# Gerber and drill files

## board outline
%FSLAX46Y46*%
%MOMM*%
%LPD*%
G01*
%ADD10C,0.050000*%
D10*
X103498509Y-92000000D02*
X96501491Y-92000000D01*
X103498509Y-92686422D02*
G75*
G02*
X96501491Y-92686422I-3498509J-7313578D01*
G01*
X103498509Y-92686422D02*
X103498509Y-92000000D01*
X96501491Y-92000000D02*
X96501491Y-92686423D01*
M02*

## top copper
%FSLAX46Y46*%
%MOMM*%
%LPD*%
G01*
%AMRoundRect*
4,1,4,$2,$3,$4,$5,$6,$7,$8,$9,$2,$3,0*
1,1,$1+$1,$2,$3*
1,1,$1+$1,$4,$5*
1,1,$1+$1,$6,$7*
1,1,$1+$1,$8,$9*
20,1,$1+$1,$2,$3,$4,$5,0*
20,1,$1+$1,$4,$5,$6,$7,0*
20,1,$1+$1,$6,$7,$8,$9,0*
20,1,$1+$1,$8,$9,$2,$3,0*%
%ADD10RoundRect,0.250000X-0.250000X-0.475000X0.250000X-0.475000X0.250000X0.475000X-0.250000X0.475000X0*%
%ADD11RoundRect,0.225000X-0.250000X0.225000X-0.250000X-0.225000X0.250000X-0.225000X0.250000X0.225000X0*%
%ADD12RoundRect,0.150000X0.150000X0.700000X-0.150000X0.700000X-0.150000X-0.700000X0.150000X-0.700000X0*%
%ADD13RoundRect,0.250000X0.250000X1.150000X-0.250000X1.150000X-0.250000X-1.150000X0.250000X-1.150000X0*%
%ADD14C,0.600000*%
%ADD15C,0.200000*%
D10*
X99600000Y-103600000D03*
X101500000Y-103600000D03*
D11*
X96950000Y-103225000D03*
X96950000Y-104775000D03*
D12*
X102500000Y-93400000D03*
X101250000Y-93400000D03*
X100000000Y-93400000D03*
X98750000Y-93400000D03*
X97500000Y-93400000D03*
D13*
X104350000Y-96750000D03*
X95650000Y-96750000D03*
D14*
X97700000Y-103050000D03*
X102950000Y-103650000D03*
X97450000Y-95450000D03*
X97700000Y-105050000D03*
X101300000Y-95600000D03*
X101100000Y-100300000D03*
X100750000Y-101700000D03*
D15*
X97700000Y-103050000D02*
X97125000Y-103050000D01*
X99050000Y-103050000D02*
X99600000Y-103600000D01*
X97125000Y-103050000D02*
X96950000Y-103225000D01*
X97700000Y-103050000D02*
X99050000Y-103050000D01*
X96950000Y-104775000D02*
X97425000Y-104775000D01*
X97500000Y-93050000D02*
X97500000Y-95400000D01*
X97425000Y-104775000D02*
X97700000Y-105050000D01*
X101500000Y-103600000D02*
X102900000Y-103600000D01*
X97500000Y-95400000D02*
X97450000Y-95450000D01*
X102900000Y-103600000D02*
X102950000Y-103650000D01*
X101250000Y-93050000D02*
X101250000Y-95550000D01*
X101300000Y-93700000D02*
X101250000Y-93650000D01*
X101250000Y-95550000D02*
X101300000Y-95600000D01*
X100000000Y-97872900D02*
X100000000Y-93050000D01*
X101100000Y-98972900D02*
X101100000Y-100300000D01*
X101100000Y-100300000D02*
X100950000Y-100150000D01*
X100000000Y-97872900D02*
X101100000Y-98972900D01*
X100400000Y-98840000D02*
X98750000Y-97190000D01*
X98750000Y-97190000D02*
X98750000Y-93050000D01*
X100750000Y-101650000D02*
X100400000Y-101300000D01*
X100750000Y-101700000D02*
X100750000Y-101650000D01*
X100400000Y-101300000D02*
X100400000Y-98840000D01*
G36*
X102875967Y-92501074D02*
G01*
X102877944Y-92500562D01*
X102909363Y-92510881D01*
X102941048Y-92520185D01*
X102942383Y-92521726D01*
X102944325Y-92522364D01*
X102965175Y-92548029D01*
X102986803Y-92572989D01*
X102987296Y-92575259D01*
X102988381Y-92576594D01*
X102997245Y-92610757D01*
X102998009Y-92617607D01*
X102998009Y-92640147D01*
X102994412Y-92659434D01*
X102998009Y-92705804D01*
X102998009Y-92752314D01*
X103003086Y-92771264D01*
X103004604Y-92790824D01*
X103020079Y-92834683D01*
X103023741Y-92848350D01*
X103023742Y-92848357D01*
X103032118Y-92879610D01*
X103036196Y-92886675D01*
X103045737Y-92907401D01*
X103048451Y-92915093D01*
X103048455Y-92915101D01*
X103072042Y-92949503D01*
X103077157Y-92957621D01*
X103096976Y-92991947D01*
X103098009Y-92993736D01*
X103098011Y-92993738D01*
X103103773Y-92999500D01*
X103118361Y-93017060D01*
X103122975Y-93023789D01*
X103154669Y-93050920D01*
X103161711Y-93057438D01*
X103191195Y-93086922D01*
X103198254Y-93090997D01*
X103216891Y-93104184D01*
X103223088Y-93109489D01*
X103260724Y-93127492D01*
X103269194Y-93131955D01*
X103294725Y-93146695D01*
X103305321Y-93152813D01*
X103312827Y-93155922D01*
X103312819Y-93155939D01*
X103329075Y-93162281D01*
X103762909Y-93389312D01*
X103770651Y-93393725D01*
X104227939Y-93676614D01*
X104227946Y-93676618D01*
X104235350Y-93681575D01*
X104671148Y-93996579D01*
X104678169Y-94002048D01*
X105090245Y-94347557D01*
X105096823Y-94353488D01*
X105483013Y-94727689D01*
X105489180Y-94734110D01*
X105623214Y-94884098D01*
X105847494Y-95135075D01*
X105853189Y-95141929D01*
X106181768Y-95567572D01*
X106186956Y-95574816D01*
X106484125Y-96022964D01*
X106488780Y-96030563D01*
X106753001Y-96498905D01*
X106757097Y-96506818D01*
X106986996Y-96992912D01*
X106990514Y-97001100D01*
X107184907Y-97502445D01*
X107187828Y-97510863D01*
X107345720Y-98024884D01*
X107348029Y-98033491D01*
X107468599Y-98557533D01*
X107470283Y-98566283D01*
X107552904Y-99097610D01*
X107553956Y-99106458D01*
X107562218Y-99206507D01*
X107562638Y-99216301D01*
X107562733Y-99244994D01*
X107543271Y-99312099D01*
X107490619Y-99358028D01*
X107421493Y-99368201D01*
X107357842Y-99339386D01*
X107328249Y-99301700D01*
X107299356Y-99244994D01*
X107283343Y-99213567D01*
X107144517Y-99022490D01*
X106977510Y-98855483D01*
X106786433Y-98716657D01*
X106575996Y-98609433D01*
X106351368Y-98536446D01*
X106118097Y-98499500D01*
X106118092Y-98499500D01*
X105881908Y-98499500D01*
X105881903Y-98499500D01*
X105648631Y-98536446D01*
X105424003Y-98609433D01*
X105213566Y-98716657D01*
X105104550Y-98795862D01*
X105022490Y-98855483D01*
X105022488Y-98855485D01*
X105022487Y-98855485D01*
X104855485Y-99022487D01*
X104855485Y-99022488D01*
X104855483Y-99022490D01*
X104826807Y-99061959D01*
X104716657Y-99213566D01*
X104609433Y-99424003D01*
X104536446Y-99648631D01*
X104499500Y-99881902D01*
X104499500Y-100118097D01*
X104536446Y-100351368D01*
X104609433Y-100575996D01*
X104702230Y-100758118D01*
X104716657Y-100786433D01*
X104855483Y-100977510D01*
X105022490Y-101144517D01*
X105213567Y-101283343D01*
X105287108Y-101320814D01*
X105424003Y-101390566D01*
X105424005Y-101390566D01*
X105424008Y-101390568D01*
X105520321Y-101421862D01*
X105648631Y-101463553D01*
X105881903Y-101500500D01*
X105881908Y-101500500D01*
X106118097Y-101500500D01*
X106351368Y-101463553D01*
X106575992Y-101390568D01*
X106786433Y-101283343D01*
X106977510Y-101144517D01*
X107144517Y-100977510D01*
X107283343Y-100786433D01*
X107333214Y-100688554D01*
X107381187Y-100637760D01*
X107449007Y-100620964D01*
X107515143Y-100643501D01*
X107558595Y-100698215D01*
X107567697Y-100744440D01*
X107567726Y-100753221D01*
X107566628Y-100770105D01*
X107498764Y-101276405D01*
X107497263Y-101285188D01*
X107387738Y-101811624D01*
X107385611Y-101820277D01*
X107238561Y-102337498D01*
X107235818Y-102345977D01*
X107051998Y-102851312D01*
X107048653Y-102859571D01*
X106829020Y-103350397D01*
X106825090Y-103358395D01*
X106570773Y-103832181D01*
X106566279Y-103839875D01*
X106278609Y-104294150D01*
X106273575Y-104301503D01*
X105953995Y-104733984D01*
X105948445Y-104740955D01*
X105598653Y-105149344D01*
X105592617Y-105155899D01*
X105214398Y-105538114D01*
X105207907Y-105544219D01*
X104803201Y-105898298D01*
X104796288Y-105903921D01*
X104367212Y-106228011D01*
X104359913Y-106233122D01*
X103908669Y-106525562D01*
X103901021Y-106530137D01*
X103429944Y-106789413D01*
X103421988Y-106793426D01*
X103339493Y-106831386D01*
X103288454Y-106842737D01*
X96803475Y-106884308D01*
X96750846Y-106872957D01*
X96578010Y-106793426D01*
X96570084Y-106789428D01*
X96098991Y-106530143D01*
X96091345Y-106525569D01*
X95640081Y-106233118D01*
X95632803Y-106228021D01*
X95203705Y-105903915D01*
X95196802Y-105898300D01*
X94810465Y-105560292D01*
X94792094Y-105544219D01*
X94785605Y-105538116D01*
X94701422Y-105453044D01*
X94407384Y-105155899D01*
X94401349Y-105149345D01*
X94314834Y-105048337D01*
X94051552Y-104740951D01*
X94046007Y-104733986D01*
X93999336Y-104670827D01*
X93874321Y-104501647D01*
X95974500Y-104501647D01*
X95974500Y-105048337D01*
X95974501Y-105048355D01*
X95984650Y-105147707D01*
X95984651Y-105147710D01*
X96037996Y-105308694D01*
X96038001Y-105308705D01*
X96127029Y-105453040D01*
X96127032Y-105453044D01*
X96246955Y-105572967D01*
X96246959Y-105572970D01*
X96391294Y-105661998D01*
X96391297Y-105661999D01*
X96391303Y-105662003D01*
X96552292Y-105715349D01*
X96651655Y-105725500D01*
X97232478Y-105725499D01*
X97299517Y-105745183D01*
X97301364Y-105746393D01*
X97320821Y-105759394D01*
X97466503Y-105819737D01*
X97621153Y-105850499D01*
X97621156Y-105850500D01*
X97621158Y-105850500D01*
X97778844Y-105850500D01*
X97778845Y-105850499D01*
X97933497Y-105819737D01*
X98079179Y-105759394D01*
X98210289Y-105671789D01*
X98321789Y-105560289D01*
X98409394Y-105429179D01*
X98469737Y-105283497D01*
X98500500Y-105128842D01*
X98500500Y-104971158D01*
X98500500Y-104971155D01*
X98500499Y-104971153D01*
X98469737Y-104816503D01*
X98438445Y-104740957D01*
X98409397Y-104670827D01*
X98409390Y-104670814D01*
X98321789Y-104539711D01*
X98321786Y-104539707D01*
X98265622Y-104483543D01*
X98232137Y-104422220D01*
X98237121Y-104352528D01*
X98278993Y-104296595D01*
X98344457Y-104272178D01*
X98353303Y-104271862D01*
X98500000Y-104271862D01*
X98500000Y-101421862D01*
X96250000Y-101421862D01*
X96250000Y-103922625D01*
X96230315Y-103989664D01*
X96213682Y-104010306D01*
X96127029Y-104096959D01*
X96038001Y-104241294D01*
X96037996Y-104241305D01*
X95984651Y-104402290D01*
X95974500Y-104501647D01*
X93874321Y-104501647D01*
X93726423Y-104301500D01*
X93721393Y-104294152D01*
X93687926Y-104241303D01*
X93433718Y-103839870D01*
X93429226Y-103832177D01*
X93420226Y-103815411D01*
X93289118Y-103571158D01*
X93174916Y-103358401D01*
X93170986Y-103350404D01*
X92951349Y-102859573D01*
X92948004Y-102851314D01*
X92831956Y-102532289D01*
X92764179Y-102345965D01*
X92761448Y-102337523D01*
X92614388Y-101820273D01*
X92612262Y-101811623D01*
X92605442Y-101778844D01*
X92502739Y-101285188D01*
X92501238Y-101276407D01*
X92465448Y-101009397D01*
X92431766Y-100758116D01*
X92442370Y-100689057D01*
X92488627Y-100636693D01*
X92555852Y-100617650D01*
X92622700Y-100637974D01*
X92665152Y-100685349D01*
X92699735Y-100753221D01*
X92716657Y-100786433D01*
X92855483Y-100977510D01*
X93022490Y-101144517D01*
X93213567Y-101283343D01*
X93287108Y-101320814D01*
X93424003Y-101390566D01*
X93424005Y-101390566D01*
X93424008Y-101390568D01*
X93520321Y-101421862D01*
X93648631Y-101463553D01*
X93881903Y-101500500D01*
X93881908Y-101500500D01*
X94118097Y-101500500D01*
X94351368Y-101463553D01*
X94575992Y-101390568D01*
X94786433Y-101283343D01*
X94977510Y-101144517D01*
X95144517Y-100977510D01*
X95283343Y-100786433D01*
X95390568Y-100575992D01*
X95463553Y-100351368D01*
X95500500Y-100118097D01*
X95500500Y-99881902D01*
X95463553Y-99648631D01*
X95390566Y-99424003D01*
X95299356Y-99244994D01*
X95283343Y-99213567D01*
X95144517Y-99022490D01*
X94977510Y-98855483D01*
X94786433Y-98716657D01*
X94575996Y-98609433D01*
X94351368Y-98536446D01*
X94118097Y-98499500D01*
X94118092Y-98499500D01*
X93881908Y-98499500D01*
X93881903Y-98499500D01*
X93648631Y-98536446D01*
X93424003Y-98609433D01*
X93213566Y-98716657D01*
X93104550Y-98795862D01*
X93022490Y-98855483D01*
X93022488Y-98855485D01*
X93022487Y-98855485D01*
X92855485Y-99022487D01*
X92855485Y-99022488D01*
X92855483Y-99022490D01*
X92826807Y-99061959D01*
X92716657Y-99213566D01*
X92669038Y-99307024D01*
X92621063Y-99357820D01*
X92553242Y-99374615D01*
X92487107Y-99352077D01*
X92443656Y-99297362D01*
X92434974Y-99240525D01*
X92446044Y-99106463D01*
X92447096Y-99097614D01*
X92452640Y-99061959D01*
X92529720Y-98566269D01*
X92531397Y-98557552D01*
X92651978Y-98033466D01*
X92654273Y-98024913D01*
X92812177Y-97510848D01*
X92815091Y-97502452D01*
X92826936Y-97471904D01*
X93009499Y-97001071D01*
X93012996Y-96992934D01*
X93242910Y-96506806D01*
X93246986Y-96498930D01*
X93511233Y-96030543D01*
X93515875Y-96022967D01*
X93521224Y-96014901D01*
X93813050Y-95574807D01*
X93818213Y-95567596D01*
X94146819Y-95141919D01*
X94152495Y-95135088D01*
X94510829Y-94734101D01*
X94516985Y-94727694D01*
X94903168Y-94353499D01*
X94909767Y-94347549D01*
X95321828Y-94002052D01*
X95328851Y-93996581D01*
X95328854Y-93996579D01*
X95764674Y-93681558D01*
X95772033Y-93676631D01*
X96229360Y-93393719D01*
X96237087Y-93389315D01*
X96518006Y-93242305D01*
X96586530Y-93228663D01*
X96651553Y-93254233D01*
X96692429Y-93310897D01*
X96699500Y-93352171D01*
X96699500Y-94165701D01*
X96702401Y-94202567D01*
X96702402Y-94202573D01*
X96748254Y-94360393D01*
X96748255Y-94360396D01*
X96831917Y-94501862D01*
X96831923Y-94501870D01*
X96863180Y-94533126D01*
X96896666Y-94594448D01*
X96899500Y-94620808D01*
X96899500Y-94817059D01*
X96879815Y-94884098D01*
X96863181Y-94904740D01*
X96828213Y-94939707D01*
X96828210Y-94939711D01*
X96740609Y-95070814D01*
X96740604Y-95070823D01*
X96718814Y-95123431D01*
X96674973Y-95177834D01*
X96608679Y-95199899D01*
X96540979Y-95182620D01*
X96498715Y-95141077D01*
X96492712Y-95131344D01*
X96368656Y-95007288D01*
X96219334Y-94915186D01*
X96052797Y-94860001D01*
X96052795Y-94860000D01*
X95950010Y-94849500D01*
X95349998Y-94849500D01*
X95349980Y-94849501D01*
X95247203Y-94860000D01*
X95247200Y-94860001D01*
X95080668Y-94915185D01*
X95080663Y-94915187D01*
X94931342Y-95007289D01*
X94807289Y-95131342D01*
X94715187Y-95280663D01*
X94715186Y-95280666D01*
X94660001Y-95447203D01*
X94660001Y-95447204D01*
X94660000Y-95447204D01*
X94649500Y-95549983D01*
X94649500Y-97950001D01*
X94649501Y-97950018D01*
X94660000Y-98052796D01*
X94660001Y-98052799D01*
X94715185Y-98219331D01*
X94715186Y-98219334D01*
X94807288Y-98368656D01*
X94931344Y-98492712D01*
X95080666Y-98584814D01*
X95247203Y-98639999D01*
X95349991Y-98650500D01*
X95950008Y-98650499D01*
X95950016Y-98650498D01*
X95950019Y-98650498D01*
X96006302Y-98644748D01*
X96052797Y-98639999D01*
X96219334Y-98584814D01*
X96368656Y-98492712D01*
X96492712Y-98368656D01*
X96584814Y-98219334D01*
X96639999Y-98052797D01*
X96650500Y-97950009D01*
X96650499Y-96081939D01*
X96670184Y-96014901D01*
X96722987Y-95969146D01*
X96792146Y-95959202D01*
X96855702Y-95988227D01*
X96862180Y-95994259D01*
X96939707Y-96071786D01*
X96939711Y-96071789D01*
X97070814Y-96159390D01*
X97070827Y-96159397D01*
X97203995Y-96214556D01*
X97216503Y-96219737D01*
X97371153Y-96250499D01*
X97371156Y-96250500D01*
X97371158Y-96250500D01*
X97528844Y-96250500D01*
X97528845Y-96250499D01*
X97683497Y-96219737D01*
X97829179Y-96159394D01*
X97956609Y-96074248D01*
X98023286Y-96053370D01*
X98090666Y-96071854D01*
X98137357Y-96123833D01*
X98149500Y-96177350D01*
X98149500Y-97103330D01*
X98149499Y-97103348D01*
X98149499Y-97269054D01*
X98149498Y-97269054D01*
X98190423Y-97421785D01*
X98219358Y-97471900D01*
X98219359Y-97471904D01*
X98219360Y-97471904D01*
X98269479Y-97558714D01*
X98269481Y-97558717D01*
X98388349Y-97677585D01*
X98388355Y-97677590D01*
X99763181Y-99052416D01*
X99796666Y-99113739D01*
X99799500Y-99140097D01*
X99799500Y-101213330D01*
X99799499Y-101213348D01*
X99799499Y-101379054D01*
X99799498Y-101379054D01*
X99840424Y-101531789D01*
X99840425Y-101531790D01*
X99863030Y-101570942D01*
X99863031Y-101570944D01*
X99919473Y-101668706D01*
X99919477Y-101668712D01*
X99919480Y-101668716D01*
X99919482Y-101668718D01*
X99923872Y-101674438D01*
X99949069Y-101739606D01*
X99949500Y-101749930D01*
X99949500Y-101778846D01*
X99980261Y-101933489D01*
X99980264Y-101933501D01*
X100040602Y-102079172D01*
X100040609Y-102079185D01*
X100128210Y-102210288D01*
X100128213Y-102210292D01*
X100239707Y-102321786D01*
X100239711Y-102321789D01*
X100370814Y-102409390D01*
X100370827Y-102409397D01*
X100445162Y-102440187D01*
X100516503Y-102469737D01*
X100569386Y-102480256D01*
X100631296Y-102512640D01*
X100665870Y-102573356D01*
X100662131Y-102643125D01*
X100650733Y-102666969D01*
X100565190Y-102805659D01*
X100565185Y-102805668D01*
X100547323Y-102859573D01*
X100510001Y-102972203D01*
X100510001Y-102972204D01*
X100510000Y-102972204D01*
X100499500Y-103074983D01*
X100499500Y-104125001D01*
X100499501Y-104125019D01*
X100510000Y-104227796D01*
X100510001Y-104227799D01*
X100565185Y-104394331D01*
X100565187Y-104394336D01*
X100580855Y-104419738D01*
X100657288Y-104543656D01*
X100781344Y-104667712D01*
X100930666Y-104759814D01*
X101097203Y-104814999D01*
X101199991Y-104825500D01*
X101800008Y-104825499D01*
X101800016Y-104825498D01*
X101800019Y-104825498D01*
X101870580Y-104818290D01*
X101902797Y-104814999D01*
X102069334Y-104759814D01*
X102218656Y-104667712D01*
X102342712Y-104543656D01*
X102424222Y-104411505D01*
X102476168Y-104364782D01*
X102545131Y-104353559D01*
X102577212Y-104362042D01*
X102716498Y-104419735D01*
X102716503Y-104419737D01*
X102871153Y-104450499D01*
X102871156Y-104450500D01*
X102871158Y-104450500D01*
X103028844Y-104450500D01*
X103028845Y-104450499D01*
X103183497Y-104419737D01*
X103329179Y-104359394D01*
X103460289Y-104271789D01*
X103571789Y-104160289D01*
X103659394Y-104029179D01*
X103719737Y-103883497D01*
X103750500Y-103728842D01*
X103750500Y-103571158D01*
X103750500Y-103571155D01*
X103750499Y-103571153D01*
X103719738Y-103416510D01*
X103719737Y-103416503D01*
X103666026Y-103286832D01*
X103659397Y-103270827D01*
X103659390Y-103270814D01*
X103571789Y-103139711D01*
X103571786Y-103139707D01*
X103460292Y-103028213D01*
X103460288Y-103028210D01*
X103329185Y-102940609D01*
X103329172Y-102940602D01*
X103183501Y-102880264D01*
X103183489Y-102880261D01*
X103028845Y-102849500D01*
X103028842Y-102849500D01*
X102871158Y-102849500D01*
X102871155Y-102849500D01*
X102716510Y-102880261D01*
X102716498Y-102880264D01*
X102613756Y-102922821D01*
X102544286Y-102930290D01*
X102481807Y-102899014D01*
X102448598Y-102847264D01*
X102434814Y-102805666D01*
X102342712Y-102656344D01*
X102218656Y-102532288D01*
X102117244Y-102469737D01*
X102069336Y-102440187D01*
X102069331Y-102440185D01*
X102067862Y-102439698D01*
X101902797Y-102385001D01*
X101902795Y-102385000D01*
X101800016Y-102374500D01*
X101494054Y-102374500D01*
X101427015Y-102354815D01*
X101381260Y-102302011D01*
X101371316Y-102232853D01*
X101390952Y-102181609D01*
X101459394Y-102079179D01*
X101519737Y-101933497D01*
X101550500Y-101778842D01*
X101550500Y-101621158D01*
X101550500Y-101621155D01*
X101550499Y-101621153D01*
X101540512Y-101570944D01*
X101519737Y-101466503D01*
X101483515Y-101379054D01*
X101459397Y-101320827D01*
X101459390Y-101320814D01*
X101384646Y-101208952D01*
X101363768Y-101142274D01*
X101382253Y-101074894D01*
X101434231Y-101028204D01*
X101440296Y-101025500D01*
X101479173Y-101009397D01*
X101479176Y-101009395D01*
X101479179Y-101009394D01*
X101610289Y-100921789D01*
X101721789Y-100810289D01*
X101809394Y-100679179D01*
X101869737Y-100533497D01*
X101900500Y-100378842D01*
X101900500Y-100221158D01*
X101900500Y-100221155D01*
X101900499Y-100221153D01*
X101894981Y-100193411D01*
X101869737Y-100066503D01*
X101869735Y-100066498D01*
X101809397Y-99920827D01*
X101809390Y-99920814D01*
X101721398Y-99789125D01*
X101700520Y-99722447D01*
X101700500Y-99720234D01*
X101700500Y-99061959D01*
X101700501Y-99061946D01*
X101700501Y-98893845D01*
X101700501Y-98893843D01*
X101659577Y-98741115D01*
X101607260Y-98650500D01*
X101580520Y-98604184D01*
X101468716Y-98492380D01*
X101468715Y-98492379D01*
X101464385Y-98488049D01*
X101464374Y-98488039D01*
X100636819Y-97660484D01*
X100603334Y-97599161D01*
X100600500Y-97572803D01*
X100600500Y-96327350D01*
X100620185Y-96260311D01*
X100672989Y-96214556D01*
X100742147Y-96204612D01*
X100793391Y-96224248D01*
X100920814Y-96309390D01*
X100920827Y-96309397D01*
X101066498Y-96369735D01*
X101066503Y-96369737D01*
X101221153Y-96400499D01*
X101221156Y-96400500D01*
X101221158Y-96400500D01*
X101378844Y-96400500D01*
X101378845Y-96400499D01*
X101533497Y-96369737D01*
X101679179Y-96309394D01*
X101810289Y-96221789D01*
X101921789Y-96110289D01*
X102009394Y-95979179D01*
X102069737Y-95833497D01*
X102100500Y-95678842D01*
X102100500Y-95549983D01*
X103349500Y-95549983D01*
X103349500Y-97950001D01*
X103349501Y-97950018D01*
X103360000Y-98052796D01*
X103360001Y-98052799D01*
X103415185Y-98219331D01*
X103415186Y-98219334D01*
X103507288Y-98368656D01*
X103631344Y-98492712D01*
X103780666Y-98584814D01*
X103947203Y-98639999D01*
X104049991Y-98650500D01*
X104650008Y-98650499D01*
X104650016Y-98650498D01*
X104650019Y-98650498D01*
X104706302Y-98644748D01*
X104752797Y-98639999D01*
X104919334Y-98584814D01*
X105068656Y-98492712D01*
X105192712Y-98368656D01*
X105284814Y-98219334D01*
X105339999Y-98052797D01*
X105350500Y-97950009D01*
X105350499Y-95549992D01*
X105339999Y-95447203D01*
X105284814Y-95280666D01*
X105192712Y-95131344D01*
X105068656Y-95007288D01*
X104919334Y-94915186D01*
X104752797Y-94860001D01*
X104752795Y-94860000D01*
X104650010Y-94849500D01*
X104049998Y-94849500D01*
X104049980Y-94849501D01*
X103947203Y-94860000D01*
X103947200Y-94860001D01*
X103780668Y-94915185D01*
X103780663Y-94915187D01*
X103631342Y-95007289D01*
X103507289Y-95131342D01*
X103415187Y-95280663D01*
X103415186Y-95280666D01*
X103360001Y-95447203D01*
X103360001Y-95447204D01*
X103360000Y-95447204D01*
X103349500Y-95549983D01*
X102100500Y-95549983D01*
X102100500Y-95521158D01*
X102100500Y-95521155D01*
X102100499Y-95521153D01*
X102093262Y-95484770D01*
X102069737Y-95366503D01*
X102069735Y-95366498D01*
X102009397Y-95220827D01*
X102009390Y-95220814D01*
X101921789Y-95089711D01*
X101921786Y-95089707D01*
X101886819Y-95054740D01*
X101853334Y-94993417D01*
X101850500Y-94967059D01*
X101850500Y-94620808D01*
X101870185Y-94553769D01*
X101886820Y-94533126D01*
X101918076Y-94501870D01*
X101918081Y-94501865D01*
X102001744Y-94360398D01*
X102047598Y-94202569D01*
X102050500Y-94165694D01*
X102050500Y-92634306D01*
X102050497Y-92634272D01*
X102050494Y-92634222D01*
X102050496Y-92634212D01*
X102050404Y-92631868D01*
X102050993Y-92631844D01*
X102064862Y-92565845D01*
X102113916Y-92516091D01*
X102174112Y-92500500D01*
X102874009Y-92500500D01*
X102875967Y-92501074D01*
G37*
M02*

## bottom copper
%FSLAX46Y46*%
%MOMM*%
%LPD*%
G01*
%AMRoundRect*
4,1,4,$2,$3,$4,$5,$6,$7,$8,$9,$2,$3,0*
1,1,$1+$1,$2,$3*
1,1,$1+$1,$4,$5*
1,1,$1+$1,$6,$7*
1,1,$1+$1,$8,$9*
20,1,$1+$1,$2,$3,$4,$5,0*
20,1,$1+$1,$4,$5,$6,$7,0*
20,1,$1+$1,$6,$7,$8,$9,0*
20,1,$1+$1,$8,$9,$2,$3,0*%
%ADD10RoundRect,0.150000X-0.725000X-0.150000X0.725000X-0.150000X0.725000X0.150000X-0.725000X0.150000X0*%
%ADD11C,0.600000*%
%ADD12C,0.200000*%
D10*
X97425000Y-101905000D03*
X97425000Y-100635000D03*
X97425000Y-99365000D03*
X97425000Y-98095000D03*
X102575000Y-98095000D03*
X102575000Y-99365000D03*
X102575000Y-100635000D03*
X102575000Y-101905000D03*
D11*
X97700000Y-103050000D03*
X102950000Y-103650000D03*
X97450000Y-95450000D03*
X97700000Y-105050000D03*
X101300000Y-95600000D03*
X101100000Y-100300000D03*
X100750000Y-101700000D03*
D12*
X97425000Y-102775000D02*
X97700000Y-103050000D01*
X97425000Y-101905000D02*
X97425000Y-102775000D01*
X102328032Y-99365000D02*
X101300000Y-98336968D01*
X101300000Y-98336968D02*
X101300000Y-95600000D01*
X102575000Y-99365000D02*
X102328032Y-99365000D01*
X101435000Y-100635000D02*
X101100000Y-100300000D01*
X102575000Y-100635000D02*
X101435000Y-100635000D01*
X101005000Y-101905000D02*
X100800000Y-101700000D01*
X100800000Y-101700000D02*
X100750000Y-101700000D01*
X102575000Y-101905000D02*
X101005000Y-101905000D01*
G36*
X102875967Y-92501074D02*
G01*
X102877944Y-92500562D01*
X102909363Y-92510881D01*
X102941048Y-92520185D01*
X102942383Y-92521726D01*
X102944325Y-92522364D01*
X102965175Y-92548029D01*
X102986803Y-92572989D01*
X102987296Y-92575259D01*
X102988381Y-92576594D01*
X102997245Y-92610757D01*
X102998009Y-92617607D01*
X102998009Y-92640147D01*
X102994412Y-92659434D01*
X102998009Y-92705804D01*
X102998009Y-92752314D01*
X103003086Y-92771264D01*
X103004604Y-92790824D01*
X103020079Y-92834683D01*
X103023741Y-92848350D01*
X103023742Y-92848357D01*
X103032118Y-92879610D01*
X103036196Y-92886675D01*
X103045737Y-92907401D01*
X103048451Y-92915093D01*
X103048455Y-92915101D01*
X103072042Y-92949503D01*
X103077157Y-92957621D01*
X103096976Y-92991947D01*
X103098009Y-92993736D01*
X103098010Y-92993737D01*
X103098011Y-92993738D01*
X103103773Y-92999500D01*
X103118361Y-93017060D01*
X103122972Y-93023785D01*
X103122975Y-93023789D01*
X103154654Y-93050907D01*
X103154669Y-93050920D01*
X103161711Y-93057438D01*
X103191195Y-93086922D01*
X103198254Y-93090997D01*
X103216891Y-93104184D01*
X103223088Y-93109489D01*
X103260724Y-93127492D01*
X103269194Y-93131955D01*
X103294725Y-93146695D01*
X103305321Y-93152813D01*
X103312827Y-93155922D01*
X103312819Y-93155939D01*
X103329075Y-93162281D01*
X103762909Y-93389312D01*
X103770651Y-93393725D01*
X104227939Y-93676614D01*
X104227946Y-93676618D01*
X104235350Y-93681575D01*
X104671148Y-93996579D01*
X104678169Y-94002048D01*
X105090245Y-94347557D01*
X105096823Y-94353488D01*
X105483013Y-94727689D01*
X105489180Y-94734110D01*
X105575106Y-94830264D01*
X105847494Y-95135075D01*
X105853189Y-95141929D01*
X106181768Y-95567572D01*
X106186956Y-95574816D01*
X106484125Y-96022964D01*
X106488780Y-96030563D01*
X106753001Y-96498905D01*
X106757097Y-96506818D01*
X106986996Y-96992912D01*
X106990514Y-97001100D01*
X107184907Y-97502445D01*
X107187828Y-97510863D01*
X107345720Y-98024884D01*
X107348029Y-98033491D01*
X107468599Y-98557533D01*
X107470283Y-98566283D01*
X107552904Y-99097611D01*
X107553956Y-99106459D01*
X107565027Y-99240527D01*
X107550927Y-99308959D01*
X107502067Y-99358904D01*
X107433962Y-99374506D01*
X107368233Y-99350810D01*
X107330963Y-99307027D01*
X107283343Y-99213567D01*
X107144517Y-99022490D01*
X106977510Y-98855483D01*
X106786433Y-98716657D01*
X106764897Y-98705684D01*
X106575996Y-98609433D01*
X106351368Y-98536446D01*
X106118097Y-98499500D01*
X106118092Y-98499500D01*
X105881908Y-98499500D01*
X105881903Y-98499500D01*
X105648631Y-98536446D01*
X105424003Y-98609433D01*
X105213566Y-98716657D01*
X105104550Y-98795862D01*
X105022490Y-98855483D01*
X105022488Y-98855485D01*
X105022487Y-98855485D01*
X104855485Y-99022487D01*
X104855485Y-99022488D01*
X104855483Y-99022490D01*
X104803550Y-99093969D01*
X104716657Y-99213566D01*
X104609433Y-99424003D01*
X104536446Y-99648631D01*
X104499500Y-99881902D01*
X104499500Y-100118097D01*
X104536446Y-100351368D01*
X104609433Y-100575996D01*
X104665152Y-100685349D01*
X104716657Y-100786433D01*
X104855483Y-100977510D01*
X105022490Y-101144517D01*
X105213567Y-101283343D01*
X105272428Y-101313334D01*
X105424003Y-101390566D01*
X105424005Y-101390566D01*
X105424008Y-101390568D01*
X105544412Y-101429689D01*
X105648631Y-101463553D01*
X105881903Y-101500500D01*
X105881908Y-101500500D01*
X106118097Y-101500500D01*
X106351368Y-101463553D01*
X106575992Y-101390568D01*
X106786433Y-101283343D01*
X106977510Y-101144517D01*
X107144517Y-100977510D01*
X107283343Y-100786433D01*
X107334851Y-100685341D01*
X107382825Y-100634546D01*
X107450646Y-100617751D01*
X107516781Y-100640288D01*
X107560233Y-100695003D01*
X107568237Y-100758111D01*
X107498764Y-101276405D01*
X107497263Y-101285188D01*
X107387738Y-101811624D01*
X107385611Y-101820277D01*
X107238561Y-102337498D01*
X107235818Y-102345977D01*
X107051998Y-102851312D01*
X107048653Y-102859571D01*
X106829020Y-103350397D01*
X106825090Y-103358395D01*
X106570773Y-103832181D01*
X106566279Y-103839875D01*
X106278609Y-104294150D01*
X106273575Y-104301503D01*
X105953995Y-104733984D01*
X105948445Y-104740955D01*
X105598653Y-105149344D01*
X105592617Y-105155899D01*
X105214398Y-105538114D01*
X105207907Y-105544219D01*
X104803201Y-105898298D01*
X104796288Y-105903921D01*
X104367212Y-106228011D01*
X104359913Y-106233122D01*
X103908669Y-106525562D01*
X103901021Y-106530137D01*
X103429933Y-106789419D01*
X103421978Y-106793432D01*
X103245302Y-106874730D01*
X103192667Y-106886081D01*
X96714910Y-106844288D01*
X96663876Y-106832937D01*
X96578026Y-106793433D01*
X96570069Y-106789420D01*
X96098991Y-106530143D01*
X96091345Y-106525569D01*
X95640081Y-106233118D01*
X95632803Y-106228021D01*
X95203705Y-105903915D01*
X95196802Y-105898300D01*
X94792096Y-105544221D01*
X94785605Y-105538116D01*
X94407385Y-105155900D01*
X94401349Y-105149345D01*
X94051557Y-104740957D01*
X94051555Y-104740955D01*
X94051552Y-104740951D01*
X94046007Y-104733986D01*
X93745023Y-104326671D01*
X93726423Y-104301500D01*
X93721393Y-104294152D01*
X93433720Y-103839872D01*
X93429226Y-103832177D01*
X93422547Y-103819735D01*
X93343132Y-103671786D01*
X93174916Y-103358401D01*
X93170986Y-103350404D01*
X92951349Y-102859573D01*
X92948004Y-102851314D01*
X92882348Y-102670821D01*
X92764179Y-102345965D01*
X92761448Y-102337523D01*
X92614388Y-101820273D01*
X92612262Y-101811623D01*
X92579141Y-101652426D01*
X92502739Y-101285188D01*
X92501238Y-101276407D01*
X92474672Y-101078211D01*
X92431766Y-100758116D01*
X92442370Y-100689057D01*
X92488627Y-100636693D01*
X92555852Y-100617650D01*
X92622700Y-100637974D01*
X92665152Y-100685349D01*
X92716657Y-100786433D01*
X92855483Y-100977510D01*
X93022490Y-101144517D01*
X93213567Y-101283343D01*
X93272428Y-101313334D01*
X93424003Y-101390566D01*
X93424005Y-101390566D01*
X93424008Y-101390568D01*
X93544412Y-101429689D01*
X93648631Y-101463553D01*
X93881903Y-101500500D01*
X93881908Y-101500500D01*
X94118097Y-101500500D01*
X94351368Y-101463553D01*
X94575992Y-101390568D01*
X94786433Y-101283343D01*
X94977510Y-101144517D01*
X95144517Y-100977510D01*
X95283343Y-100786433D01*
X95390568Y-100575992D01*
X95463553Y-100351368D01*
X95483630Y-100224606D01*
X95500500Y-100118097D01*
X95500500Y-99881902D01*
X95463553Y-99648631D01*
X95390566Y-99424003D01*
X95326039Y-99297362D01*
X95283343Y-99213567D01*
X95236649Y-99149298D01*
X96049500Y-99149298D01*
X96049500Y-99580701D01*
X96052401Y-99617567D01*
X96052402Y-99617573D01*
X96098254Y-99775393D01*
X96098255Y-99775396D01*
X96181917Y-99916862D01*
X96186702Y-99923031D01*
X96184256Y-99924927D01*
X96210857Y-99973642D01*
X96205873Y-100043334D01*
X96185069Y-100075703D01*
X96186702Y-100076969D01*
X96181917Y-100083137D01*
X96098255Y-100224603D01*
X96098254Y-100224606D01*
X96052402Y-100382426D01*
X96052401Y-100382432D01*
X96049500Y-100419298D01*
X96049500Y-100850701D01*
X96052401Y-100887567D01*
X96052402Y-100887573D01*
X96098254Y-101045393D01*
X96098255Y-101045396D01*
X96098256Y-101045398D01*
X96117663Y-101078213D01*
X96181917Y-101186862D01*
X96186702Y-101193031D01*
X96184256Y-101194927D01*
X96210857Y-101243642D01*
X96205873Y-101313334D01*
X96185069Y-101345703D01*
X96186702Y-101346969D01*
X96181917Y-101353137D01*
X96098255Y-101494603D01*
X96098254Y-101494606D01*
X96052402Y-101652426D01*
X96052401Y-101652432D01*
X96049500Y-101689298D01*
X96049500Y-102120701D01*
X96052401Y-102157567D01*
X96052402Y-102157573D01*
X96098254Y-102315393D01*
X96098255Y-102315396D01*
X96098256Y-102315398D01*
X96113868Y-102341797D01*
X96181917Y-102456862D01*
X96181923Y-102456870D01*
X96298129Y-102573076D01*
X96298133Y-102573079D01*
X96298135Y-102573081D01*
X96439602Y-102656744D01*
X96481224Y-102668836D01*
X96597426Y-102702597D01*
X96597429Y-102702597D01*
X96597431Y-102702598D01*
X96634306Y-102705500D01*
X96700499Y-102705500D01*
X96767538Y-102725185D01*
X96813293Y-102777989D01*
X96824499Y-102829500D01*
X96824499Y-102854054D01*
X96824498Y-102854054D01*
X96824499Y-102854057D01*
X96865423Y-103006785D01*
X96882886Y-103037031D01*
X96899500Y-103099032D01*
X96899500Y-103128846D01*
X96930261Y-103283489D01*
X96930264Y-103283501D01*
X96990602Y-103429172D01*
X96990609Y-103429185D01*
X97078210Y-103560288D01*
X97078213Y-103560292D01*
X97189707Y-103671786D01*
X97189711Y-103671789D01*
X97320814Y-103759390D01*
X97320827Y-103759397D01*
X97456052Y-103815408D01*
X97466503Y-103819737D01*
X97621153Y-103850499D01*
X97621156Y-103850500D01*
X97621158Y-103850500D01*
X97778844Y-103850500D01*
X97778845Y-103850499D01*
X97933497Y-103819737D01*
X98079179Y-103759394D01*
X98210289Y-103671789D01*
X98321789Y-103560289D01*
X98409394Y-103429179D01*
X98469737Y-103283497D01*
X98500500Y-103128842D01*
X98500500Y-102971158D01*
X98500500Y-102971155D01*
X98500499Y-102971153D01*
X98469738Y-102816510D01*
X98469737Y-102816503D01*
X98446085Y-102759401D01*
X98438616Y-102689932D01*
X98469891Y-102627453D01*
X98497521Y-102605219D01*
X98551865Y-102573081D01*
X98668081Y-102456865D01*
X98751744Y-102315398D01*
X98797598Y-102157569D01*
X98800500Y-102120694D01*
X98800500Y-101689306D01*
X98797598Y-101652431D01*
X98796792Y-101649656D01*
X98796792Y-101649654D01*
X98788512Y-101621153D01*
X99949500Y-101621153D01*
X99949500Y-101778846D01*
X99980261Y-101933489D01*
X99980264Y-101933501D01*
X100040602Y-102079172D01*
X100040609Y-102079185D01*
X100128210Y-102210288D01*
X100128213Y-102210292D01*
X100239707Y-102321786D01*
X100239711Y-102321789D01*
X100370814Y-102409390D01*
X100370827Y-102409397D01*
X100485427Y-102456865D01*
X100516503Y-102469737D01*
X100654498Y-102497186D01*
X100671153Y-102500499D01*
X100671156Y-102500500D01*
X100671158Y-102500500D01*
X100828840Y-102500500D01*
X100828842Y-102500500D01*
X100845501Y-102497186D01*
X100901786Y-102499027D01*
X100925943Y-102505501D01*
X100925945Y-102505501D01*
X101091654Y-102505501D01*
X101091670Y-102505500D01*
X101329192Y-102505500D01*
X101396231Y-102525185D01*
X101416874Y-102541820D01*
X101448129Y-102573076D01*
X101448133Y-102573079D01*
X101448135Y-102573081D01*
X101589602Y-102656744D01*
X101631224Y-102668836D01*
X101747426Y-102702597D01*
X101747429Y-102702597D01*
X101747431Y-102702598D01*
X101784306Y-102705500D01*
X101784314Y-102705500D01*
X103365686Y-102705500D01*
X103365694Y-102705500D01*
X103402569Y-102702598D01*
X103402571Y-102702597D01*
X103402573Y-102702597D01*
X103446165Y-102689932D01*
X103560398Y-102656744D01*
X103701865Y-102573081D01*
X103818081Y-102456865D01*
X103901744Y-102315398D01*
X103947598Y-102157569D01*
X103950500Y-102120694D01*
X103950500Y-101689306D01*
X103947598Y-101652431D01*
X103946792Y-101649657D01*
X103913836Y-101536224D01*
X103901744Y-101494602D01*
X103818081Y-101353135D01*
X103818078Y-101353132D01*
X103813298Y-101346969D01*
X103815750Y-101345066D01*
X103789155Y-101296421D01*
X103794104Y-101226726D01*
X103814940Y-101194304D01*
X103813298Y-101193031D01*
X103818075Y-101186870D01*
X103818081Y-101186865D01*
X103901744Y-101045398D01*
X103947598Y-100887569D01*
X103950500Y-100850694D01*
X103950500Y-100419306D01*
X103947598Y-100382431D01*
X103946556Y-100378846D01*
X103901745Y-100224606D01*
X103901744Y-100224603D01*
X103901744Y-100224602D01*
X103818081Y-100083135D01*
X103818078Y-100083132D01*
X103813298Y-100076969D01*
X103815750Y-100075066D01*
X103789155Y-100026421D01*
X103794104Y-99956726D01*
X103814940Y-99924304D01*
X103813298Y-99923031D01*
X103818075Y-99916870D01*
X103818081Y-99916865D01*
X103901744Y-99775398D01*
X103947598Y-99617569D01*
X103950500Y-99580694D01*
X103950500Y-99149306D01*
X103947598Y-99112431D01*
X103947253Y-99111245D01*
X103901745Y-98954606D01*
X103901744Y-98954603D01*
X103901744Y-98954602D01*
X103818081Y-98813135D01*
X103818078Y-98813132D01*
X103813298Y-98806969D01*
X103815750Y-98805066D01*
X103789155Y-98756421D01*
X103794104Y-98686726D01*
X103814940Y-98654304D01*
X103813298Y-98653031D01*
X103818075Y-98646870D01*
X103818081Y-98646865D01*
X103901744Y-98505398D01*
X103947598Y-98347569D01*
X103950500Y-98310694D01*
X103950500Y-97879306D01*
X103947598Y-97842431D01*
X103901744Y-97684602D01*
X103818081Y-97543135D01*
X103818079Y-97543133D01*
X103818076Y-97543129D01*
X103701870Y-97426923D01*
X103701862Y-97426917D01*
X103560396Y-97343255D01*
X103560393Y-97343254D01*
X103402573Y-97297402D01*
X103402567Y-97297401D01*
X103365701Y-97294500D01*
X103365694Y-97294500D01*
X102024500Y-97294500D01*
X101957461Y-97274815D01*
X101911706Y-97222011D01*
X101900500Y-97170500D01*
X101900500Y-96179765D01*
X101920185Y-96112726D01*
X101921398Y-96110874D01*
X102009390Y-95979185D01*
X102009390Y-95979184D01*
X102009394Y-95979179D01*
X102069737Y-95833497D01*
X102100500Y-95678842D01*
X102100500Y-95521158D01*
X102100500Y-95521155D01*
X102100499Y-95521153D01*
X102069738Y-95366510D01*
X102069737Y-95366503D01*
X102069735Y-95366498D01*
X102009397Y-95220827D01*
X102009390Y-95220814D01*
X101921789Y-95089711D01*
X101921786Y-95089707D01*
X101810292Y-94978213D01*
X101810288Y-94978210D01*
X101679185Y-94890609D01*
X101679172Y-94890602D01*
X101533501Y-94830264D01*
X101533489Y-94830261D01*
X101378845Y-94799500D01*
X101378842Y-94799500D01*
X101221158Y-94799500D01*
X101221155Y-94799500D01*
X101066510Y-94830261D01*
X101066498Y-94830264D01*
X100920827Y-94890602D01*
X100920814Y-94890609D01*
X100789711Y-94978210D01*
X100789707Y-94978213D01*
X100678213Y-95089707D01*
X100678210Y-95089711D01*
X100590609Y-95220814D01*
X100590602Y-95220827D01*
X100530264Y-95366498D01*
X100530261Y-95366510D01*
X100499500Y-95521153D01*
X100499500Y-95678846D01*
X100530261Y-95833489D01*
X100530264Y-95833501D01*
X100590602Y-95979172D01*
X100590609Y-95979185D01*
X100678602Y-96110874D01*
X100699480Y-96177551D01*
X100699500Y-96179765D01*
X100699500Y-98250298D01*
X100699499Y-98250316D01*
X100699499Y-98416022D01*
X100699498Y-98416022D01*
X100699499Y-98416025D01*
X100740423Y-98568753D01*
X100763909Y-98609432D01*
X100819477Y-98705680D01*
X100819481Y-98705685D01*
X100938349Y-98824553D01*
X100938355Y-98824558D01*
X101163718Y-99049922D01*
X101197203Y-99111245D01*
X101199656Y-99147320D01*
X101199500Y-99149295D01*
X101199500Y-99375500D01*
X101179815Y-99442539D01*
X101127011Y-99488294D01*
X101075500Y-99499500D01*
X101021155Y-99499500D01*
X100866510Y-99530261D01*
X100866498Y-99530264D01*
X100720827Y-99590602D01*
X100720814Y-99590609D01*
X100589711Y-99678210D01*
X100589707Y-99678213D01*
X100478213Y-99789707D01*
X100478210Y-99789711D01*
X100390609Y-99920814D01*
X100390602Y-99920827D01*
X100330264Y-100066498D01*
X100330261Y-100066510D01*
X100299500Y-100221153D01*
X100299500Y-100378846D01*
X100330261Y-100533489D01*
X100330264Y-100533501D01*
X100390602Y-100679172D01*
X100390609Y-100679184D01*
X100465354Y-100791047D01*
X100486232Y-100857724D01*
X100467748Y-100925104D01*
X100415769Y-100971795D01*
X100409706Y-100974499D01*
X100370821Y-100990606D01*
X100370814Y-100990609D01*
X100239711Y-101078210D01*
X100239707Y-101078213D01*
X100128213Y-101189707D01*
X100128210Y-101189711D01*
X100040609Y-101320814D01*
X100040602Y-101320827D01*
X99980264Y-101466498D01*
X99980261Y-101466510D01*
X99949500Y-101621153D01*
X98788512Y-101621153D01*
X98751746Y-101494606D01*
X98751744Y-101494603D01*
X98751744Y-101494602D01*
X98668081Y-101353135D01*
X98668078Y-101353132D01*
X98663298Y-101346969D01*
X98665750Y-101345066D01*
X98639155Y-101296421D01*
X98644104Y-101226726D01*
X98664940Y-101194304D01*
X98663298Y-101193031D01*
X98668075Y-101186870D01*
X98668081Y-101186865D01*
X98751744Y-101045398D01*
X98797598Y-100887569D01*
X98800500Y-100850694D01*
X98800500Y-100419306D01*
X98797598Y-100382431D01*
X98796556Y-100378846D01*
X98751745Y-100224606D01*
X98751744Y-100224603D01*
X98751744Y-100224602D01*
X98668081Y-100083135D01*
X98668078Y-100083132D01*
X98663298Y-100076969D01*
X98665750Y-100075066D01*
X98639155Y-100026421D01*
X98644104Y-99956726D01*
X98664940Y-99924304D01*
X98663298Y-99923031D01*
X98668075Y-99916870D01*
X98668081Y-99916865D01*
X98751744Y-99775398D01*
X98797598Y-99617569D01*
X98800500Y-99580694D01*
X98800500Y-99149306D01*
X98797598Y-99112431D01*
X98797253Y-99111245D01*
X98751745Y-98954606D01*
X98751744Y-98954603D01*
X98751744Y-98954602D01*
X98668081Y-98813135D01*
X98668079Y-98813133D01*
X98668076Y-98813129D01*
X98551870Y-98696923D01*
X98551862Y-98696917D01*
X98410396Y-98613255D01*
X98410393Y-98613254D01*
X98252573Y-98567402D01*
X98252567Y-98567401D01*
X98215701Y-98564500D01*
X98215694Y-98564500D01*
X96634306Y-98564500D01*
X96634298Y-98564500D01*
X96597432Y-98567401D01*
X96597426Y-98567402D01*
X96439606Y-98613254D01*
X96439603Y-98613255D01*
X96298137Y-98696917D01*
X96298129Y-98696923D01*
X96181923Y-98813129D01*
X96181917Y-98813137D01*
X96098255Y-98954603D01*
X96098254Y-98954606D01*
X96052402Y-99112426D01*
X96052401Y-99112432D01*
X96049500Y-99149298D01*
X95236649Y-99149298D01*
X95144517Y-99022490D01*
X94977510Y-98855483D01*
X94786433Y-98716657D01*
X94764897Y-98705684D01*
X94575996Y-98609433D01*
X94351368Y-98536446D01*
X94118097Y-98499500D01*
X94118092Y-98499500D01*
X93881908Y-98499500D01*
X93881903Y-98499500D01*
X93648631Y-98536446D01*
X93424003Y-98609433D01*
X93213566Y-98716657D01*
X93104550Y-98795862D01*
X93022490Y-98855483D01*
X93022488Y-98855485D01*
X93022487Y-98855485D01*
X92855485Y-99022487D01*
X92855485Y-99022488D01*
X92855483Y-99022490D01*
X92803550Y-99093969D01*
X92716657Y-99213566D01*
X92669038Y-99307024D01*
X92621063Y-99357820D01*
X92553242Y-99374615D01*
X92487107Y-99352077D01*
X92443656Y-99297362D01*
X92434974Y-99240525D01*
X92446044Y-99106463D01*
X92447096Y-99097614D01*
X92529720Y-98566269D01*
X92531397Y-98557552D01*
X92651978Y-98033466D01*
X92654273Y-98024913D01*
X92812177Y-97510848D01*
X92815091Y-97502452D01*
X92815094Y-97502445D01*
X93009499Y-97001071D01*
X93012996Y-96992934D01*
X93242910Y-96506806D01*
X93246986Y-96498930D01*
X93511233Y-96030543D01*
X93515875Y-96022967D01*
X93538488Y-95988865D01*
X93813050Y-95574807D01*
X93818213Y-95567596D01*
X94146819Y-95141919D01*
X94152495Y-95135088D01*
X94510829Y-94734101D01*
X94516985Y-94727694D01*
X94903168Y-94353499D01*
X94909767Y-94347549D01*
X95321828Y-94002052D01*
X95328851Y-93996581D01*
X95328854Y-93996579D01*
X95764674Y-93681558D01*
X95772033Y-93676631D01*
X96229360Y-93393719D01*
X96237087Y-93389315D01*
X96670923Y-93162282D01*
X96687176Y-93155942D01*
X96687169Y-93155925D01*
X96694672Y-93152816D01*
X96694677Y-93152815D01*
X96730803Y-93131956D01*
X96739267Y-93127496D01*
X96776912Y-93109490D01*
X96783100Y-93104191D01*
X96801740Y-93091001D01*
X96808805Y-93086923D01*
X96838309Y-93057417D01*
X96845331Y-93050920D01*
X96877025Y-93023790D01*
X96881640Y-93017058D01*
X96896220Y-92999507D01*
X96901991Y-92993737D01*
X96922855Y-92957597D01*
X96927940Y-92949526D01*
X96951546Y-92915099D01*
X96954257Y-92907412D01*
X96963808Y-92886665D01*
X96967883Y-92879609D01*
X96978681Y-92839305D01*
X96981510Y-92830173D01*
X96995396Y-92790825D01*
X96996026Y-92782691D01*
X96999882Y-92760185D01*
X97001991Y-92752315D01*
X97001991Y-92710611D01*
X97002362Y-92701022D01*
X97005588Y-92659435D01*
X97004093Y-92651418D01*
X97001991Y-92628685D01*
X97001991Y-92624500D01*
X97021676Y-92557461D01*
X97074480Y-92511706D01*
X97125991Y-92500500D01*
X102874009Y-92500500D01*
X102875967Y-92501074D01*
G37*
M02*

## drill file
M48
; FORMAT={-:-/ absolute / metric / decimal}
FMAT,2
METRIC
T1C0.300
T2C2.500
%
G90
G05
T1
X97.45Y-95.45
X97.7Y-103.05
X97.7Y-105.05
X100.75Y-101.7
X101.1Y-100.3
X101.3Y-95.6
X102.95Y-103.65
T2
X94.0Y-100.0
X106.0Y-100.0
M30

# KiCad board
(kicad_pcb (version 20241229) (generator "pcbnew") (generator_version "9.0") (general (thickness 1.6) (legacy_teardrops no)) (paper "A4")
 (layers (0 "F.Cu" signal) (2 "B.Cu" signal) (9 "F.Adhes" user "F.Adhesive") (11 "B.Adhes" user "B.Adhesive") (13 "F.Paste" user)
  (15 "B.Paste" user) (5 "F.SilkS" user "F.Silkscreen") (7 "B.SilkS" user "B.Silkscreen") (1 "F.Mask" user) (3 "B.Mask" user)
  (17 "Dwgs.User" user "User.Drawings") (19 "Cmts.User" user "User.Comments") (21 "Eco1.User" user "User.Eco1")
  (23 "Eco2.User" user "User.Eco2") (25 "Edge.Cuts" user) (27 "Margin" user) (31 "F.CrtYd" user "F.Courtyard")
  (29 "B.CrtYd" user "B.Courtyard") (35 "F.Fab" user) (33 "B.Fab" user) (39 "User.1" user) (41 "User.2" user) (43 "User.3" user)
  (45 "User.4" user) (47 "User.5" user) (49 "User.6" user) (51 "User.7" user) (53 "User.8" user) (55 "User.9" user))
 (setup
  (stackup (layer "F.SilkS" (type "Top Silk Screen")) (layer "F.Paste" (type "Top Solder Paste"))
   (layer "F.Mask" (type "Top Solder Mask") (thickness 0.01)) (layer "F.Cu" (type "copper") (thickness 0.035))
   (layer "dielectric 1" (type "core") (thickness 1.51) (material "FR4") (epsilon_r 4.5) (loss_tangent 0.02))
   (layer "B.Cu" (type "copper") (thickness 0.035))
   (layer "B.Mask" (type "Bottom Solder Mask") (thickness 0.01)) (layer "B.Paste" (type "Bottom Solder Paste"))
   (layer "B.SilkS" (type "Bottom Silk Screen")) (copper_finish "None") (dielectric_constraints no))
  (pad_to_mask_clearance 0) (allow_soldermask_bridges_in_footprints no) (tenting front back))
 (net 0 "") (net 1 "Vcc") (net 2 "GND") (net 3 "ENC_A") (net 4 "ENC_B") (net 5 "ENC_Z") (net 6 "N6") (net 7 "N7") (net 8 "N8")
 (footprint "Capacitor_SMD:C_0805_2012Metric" (layer "F.Cu") (at 100.55 103.6)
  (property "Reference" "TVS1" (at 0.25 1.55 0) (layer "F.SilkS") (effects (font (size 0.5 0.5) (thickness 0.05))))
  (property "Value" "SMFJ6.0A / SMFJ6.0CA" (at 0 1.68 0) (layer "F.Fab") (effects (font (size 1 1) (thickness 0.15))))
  (pad "1" smd roundrect (at -0.95 0) (size 1 1.45) (layers "F.Cu" "F.Mask" "F.Paste") (roundrect_rratio 0.25) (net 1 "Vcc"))
  (pad "2" smd roundrect (at 0.95 0) (size 1 1.45) (layers "F.Cu" "F.Mask" "F.Paste") (roundrect_rratio 0.25) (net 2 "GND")))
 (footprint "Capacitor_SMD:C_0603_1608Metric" (layer "F.Cu") (at 96.95 104 -90)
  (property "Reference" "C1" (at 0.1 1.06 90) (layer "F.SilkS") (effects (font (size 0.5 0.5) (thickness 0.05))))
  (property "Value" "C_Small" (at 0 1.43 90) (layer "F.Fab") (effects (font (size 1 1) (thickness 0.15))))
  (pad "1" smd roundrect (at -0.775 0 270) (size 0.9 0.95) (layers "F.Cu" "F.Mask" "F.Paste") (roundrect_rratio 0.25) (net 1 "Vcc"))
  (pad "2" smd roundrect (at 0.775 0 270) (size 0.9 0.95) (layers "F.Cu" "F.Mask" "F.Paste") (roundrect_rratio 0.25) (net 2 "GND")))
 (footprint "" (layer "F.Cu") (at 94 100)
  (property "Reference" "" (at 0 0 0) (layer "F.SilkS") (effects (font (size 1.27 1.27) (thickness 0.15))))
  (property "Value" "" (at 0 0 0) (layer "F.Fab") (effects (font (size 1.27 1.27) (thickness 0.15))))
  (pad "" np_thru_hole circle (at 0 0) (size 2.5 2.5) (drill 2.5) (layers "*.Cu" "*.Mask")))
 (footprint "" (layer "F.Cu") (at 106 100)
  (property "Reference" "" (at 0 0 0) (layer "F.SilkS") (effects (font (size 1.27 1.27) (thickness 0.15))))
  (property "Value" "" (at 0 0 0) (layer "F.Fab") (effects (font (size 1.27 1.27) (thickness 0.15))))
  (pad "" np_thru_hole circle (at 0 0) (size 2.5 2.5) (drill 2.5) (layers "*.Cu" "*.Mask")))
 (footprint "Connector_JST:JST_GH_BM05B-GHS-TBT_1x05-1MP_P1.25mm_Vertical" (layer "F.Cu") (at 100 95.35 180)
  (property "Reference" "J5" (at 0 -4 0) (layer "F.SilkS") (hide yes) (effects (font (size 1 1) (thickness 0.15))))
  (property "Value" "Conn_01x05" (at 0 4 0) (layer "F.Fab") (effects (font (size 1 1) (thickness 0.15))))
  (pad "1" smd roundrect (at -2.5 1.95 180) (size 0.6 1.7) (layers "F.Cu" "F.Mask" "F.Paste") (roundrect_rratio 0.25) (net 1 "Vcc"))
  (pad "2" smd roundrect (at -1.25 1.95 180) (size 0.6 1.7) (layers "F.Cu" "F.Mask" "F.Paste") (roundrect_rratio 0.25) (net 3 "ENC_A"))
  (pad "3" smd roundrect (at 0 1.95 180) (size 0.6 1.7) (layers "F.Cu" "F.Mask" "F.Paste") (roundrect_rratio 0.25) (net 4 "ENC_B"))
  (pad "4" smd roundrect (at 1.25 1.95 180) (size 0.6 1.7) (layers "F.Cu" "F.Mask" "F.Paste") (roundrect_rratio 0.25) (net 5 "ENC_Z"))
  (pad "5" smd roundrect (at 2.5 1.95 180) (size 0.6 1.7) (layers "F.Cu" "F.Mask" "F.Paste") (roundrect_rratio 0.25) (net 2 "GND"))
  (pad "MP" smd roundrect (at -4.35 -1.4 180) (size 1 2.8) (layers "F.Cu" "F.Mask" "F.Paste") (roundrect_rratio 0.25))
  (pad "MP" smd roundrect (at 4.35 -1.4 180) (size 1 2.8) (layers "F.Cu" "F.Mask" "F.Paste") (roundrect_rratio 0.25)))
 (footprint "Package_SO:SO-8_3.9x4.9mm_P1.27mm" (layer "B.Cu") (at 100 100)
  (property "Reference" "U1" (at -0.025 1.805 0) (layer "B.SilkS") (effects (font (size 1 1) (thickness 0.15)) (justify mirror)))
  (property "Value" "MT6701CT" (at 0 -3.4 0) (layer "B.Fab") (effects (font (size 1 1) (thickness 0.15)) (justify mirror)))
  (pad "1" smd roundrect (at -2.575 1.905) (size 1.75 0.6) (layers "B.Cu" "B.Mask" "B.Paste") (roundrect_rratio 0.25) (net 1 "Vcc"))
  (pad "2" smd roundrect (at -2.575 0.635) (size 1.75 0.6) (layers "B.Cu" "B.Mask" "B.Paste") (roundrect_rratio 0.25) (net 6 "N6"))
  (pad "3" smd roundrect (at -2.575 -0.635) (size 1.75 0.6) (layers "B.Cu" "B.Mask" "B.Paste") (roundrect_rratio 0.25) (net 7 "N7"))
  (pad "4" smd roundrect (at -2.575 -1.905) (size 1.75 0.6) (layers "B.Cu" "B.Mask" "B.Paste") (roundrect_rratio 0.25) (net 2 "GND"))
  (pad "5" smd roundrect (at 2.575 -1.905) (size 1.75 0.6) (layers "B.Cu" "B.Mask" "B.Paste") (roundrect_rratio 0.25) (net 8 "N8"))
  (pad "6" smd roundrect (at 2.575 -0.635) (size 1.75 0.6) (layers "B.Cu" "B.Mask" "B.Paste") (roundrect_rratio 0.25) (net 3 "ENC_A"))
  (pad "7" smd roundrect (at 2.575 0.635) (size 1.75 0.6) (layers "B.Cu" "B.Mask" "B.Paste") (roundrect_rratio 0.25) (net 4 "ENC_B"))
  (pad "8" smd roundrect (at 2.575 1.905) (size 1.75 0.6) (layers "B.Cu" "B.Mask" "B.Paste") (roundrect_rratio 0.25) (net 5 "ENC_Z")))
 (gr_line (start 103.498509 92) (end 96.501491 92) (stroke (width 0.05) (type solid)) (layer "Edge.Cuts"))
 (gr_arc (start 103.498509 92.686422) (mid 100 108.107278) (end 96.501491 92.686423) (stroke (width 0.05) (type default))
  (layer "Edge.Cuts"))
 (gr_line (start 103.498509 92.686422) (end 103.498509 92) (stroke (width 0.05) (type default)) (layer "Edge.Cuts"))
 (gr_line (start 96.501491 92) (end 96.501491 92.686423) (stroke (width 0.05) (type default)) (layer "Edge.Cuts"))
 (segment (start 97.7 103.05) (end 97.125 103.05) (width 0.2) (layer "F.Cu") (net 1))
 (segment (start 99.05 103.05) (end 99.6 103.6) (width 0.2) (layer "F.Cu") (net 1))
 (segment (start 97.125 103.05) (end 96.95 103.225) (width 0.2) (layer "F.Cu") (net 1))
 (segment (start 97.7 103.05) (end 99.05 103.05) (width 0.2) (layer "F.Cu") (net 1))
 (via (at 97.7 103.05) (size 0.6) (drill 0.3) (layers "F.Cu" "B.Cu") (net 1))
 (segment (start 97.425 102.775) (end 97.7 103.05) (width 0.2) (layer "B.Cu") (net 1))
 (segment (start 97.425 101.905) (end 97.425 102.775) (width 0.2) (layer "B.Cu") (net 1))
 (segment (start 96.95 104.775) (end 97.425 104.775) (width 0.2) (layer "F.Cu") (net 2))
 (segment (start 97.5 93.05) (end 97.5 95.4) (width 0.2) (layer "F.Cu") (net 2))
 (segment (start 97.425 104.775) (end 97.7 105.05) (width 0.2) (layer "F.Cu") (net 2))
 (segment (start 101.5 103.6) (end 102.9 103.6) (width 0.2) (layer "F.Cu") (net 2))
 (segment (start 97.5 95.4) (end 97.45 95.45) (width 0.2) (layer "F.Cu") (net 2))
 (segment (start 102.9 103.6) (end 102.95 103.65) (width 0.2) (layer "F.Cu") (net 2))
 (via (at 102.95 103.65) (size 0.6) (drill 0.3) (layers "F.Cu" "B.Cu") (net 2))
 (via (at 97.45 95.45) (size 0.6) (drill 0.3) (layers "F.Cu" "B.Cu") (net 2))
 (via (at 97.7 105.05) (size 0.6) (drill 0.3) (layers "F.Cu" "B.Cu") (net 2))
 (segment (start 101.25 93.05) (end 101.25 95.55) (width 0.2) (layer "F.Cu") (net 3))
 (segment (start 101.3 93.7) (end 101.25 93.65) (width 0.2) (layer "F.Cu") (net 3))
 (segment (start 101.25 95.55) (end 101.3 95.6) (width 0.2) (layer "F.Cu") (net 3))
 (via (at 101.3 95.6) (size 0.6) (drill 0.3) (layers "F.Cu" "B.Cu") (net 3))
 (segment (start 102.328032 99.365) (end 101.3 98.336968) (width 0.2) (layer "B.Cu") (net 3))
 (segment (start 101.3 98.336968) (end 101.3 95.6) (width 0.2) (layer "B.Cu") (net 3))
 (segment (start 102.575 99.365) (end 102.328032 99.365) (width 0.2) (layer "B.Cu") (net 3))
 (segment (start 100 97.8729) (end 100 93.05) (width 0.2) (layer "F.Cu") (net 4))
 (segment (start 101.1 98.9729) (end 101.1 100.3) (width 0.2) (layer "F.Cu") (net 4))
 (segment (start 101.1 100.3) (end 100.95 100.15) (width 0.2) (layer "F.Cu") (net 4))
 (segment (start 100 97.8729) (end 101.1 98.9729) (width 0.2) (layer "F.Cu") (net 4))
 (via (at 101.1 100.3) (size 0.6) (drill 0.3) (layers "F.Cu" "B.Cu") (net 4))
 (segment (start 101.435 100.635) (end 101.1 100.3) (width 0.2) (layer "B.Cu") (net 4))
 (segment (start 102.575 100.635) (end 101.435 100.635) (width 0.2) (layer "B.Cu") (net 4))
 (segment (start 100.4 98.84) (end 98.75 97.19) (width 0.2) (layer "F.Cu") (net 5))
 (segment (start 98.75 97.19) (end 98.75 93.05) (width 0.2) (layer "F.Cu") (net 5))
 (segment (start 100.75 101.65) (end 100.4 101.3) (width 0.2) (layer "F.Cu") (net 5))
 (segment (start 100.75 101.7) (end 100.75 101.65) (width 0.2) (layer "F.Cu") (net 5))
 (segment (start 100.4 101.3) (end 100.4 98.84) (width 0.2) (layer "F.Cu") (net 5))
 (via (at 100.75 101.7) (size 0.6) (drill 0.3) (layers "F.Cu" "B.Cu") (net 5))
 (segment (start 101.005 101.905) (end 100.8 101.7) (width 0.2) (layer "B.Cu") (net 5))
 (segment (start 100.8 101.7) (end 100.75 101.7) (width 0.2) (layer "B.Cu") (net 5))
 (segment (start 102.575 101.905) (end 101.005 101.905) (width 0.2) (layer "B.Cu") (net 5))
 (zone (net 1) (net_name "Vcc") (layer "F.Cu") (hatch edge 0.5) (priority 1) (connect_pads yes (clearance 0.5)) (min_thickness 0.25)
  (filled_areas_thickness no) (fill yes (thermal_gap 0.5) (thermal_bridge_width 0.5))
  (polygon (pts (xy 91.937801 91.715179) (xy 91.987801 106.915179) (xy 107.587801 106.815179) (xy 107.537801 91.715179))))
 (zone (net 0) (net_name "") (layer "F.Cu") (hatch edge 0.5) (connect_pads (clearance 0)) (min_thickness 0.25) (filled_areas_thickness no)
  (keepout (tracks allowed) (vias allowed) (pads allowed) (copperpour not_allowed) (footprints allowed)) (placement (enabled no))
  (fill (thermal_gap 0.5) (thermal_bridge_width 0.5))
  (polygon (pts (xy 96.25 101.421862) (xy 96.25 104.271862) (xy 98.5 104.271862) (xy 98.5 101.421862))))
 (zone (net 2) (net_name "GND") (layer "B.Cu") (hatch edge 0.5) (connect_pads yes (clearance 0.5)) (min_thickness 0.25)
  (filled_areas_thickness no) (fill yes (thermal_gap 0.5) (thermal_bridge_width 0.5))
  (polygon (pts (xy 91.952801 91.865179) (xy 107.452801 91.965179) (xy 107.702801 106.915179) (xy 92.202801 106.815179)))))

